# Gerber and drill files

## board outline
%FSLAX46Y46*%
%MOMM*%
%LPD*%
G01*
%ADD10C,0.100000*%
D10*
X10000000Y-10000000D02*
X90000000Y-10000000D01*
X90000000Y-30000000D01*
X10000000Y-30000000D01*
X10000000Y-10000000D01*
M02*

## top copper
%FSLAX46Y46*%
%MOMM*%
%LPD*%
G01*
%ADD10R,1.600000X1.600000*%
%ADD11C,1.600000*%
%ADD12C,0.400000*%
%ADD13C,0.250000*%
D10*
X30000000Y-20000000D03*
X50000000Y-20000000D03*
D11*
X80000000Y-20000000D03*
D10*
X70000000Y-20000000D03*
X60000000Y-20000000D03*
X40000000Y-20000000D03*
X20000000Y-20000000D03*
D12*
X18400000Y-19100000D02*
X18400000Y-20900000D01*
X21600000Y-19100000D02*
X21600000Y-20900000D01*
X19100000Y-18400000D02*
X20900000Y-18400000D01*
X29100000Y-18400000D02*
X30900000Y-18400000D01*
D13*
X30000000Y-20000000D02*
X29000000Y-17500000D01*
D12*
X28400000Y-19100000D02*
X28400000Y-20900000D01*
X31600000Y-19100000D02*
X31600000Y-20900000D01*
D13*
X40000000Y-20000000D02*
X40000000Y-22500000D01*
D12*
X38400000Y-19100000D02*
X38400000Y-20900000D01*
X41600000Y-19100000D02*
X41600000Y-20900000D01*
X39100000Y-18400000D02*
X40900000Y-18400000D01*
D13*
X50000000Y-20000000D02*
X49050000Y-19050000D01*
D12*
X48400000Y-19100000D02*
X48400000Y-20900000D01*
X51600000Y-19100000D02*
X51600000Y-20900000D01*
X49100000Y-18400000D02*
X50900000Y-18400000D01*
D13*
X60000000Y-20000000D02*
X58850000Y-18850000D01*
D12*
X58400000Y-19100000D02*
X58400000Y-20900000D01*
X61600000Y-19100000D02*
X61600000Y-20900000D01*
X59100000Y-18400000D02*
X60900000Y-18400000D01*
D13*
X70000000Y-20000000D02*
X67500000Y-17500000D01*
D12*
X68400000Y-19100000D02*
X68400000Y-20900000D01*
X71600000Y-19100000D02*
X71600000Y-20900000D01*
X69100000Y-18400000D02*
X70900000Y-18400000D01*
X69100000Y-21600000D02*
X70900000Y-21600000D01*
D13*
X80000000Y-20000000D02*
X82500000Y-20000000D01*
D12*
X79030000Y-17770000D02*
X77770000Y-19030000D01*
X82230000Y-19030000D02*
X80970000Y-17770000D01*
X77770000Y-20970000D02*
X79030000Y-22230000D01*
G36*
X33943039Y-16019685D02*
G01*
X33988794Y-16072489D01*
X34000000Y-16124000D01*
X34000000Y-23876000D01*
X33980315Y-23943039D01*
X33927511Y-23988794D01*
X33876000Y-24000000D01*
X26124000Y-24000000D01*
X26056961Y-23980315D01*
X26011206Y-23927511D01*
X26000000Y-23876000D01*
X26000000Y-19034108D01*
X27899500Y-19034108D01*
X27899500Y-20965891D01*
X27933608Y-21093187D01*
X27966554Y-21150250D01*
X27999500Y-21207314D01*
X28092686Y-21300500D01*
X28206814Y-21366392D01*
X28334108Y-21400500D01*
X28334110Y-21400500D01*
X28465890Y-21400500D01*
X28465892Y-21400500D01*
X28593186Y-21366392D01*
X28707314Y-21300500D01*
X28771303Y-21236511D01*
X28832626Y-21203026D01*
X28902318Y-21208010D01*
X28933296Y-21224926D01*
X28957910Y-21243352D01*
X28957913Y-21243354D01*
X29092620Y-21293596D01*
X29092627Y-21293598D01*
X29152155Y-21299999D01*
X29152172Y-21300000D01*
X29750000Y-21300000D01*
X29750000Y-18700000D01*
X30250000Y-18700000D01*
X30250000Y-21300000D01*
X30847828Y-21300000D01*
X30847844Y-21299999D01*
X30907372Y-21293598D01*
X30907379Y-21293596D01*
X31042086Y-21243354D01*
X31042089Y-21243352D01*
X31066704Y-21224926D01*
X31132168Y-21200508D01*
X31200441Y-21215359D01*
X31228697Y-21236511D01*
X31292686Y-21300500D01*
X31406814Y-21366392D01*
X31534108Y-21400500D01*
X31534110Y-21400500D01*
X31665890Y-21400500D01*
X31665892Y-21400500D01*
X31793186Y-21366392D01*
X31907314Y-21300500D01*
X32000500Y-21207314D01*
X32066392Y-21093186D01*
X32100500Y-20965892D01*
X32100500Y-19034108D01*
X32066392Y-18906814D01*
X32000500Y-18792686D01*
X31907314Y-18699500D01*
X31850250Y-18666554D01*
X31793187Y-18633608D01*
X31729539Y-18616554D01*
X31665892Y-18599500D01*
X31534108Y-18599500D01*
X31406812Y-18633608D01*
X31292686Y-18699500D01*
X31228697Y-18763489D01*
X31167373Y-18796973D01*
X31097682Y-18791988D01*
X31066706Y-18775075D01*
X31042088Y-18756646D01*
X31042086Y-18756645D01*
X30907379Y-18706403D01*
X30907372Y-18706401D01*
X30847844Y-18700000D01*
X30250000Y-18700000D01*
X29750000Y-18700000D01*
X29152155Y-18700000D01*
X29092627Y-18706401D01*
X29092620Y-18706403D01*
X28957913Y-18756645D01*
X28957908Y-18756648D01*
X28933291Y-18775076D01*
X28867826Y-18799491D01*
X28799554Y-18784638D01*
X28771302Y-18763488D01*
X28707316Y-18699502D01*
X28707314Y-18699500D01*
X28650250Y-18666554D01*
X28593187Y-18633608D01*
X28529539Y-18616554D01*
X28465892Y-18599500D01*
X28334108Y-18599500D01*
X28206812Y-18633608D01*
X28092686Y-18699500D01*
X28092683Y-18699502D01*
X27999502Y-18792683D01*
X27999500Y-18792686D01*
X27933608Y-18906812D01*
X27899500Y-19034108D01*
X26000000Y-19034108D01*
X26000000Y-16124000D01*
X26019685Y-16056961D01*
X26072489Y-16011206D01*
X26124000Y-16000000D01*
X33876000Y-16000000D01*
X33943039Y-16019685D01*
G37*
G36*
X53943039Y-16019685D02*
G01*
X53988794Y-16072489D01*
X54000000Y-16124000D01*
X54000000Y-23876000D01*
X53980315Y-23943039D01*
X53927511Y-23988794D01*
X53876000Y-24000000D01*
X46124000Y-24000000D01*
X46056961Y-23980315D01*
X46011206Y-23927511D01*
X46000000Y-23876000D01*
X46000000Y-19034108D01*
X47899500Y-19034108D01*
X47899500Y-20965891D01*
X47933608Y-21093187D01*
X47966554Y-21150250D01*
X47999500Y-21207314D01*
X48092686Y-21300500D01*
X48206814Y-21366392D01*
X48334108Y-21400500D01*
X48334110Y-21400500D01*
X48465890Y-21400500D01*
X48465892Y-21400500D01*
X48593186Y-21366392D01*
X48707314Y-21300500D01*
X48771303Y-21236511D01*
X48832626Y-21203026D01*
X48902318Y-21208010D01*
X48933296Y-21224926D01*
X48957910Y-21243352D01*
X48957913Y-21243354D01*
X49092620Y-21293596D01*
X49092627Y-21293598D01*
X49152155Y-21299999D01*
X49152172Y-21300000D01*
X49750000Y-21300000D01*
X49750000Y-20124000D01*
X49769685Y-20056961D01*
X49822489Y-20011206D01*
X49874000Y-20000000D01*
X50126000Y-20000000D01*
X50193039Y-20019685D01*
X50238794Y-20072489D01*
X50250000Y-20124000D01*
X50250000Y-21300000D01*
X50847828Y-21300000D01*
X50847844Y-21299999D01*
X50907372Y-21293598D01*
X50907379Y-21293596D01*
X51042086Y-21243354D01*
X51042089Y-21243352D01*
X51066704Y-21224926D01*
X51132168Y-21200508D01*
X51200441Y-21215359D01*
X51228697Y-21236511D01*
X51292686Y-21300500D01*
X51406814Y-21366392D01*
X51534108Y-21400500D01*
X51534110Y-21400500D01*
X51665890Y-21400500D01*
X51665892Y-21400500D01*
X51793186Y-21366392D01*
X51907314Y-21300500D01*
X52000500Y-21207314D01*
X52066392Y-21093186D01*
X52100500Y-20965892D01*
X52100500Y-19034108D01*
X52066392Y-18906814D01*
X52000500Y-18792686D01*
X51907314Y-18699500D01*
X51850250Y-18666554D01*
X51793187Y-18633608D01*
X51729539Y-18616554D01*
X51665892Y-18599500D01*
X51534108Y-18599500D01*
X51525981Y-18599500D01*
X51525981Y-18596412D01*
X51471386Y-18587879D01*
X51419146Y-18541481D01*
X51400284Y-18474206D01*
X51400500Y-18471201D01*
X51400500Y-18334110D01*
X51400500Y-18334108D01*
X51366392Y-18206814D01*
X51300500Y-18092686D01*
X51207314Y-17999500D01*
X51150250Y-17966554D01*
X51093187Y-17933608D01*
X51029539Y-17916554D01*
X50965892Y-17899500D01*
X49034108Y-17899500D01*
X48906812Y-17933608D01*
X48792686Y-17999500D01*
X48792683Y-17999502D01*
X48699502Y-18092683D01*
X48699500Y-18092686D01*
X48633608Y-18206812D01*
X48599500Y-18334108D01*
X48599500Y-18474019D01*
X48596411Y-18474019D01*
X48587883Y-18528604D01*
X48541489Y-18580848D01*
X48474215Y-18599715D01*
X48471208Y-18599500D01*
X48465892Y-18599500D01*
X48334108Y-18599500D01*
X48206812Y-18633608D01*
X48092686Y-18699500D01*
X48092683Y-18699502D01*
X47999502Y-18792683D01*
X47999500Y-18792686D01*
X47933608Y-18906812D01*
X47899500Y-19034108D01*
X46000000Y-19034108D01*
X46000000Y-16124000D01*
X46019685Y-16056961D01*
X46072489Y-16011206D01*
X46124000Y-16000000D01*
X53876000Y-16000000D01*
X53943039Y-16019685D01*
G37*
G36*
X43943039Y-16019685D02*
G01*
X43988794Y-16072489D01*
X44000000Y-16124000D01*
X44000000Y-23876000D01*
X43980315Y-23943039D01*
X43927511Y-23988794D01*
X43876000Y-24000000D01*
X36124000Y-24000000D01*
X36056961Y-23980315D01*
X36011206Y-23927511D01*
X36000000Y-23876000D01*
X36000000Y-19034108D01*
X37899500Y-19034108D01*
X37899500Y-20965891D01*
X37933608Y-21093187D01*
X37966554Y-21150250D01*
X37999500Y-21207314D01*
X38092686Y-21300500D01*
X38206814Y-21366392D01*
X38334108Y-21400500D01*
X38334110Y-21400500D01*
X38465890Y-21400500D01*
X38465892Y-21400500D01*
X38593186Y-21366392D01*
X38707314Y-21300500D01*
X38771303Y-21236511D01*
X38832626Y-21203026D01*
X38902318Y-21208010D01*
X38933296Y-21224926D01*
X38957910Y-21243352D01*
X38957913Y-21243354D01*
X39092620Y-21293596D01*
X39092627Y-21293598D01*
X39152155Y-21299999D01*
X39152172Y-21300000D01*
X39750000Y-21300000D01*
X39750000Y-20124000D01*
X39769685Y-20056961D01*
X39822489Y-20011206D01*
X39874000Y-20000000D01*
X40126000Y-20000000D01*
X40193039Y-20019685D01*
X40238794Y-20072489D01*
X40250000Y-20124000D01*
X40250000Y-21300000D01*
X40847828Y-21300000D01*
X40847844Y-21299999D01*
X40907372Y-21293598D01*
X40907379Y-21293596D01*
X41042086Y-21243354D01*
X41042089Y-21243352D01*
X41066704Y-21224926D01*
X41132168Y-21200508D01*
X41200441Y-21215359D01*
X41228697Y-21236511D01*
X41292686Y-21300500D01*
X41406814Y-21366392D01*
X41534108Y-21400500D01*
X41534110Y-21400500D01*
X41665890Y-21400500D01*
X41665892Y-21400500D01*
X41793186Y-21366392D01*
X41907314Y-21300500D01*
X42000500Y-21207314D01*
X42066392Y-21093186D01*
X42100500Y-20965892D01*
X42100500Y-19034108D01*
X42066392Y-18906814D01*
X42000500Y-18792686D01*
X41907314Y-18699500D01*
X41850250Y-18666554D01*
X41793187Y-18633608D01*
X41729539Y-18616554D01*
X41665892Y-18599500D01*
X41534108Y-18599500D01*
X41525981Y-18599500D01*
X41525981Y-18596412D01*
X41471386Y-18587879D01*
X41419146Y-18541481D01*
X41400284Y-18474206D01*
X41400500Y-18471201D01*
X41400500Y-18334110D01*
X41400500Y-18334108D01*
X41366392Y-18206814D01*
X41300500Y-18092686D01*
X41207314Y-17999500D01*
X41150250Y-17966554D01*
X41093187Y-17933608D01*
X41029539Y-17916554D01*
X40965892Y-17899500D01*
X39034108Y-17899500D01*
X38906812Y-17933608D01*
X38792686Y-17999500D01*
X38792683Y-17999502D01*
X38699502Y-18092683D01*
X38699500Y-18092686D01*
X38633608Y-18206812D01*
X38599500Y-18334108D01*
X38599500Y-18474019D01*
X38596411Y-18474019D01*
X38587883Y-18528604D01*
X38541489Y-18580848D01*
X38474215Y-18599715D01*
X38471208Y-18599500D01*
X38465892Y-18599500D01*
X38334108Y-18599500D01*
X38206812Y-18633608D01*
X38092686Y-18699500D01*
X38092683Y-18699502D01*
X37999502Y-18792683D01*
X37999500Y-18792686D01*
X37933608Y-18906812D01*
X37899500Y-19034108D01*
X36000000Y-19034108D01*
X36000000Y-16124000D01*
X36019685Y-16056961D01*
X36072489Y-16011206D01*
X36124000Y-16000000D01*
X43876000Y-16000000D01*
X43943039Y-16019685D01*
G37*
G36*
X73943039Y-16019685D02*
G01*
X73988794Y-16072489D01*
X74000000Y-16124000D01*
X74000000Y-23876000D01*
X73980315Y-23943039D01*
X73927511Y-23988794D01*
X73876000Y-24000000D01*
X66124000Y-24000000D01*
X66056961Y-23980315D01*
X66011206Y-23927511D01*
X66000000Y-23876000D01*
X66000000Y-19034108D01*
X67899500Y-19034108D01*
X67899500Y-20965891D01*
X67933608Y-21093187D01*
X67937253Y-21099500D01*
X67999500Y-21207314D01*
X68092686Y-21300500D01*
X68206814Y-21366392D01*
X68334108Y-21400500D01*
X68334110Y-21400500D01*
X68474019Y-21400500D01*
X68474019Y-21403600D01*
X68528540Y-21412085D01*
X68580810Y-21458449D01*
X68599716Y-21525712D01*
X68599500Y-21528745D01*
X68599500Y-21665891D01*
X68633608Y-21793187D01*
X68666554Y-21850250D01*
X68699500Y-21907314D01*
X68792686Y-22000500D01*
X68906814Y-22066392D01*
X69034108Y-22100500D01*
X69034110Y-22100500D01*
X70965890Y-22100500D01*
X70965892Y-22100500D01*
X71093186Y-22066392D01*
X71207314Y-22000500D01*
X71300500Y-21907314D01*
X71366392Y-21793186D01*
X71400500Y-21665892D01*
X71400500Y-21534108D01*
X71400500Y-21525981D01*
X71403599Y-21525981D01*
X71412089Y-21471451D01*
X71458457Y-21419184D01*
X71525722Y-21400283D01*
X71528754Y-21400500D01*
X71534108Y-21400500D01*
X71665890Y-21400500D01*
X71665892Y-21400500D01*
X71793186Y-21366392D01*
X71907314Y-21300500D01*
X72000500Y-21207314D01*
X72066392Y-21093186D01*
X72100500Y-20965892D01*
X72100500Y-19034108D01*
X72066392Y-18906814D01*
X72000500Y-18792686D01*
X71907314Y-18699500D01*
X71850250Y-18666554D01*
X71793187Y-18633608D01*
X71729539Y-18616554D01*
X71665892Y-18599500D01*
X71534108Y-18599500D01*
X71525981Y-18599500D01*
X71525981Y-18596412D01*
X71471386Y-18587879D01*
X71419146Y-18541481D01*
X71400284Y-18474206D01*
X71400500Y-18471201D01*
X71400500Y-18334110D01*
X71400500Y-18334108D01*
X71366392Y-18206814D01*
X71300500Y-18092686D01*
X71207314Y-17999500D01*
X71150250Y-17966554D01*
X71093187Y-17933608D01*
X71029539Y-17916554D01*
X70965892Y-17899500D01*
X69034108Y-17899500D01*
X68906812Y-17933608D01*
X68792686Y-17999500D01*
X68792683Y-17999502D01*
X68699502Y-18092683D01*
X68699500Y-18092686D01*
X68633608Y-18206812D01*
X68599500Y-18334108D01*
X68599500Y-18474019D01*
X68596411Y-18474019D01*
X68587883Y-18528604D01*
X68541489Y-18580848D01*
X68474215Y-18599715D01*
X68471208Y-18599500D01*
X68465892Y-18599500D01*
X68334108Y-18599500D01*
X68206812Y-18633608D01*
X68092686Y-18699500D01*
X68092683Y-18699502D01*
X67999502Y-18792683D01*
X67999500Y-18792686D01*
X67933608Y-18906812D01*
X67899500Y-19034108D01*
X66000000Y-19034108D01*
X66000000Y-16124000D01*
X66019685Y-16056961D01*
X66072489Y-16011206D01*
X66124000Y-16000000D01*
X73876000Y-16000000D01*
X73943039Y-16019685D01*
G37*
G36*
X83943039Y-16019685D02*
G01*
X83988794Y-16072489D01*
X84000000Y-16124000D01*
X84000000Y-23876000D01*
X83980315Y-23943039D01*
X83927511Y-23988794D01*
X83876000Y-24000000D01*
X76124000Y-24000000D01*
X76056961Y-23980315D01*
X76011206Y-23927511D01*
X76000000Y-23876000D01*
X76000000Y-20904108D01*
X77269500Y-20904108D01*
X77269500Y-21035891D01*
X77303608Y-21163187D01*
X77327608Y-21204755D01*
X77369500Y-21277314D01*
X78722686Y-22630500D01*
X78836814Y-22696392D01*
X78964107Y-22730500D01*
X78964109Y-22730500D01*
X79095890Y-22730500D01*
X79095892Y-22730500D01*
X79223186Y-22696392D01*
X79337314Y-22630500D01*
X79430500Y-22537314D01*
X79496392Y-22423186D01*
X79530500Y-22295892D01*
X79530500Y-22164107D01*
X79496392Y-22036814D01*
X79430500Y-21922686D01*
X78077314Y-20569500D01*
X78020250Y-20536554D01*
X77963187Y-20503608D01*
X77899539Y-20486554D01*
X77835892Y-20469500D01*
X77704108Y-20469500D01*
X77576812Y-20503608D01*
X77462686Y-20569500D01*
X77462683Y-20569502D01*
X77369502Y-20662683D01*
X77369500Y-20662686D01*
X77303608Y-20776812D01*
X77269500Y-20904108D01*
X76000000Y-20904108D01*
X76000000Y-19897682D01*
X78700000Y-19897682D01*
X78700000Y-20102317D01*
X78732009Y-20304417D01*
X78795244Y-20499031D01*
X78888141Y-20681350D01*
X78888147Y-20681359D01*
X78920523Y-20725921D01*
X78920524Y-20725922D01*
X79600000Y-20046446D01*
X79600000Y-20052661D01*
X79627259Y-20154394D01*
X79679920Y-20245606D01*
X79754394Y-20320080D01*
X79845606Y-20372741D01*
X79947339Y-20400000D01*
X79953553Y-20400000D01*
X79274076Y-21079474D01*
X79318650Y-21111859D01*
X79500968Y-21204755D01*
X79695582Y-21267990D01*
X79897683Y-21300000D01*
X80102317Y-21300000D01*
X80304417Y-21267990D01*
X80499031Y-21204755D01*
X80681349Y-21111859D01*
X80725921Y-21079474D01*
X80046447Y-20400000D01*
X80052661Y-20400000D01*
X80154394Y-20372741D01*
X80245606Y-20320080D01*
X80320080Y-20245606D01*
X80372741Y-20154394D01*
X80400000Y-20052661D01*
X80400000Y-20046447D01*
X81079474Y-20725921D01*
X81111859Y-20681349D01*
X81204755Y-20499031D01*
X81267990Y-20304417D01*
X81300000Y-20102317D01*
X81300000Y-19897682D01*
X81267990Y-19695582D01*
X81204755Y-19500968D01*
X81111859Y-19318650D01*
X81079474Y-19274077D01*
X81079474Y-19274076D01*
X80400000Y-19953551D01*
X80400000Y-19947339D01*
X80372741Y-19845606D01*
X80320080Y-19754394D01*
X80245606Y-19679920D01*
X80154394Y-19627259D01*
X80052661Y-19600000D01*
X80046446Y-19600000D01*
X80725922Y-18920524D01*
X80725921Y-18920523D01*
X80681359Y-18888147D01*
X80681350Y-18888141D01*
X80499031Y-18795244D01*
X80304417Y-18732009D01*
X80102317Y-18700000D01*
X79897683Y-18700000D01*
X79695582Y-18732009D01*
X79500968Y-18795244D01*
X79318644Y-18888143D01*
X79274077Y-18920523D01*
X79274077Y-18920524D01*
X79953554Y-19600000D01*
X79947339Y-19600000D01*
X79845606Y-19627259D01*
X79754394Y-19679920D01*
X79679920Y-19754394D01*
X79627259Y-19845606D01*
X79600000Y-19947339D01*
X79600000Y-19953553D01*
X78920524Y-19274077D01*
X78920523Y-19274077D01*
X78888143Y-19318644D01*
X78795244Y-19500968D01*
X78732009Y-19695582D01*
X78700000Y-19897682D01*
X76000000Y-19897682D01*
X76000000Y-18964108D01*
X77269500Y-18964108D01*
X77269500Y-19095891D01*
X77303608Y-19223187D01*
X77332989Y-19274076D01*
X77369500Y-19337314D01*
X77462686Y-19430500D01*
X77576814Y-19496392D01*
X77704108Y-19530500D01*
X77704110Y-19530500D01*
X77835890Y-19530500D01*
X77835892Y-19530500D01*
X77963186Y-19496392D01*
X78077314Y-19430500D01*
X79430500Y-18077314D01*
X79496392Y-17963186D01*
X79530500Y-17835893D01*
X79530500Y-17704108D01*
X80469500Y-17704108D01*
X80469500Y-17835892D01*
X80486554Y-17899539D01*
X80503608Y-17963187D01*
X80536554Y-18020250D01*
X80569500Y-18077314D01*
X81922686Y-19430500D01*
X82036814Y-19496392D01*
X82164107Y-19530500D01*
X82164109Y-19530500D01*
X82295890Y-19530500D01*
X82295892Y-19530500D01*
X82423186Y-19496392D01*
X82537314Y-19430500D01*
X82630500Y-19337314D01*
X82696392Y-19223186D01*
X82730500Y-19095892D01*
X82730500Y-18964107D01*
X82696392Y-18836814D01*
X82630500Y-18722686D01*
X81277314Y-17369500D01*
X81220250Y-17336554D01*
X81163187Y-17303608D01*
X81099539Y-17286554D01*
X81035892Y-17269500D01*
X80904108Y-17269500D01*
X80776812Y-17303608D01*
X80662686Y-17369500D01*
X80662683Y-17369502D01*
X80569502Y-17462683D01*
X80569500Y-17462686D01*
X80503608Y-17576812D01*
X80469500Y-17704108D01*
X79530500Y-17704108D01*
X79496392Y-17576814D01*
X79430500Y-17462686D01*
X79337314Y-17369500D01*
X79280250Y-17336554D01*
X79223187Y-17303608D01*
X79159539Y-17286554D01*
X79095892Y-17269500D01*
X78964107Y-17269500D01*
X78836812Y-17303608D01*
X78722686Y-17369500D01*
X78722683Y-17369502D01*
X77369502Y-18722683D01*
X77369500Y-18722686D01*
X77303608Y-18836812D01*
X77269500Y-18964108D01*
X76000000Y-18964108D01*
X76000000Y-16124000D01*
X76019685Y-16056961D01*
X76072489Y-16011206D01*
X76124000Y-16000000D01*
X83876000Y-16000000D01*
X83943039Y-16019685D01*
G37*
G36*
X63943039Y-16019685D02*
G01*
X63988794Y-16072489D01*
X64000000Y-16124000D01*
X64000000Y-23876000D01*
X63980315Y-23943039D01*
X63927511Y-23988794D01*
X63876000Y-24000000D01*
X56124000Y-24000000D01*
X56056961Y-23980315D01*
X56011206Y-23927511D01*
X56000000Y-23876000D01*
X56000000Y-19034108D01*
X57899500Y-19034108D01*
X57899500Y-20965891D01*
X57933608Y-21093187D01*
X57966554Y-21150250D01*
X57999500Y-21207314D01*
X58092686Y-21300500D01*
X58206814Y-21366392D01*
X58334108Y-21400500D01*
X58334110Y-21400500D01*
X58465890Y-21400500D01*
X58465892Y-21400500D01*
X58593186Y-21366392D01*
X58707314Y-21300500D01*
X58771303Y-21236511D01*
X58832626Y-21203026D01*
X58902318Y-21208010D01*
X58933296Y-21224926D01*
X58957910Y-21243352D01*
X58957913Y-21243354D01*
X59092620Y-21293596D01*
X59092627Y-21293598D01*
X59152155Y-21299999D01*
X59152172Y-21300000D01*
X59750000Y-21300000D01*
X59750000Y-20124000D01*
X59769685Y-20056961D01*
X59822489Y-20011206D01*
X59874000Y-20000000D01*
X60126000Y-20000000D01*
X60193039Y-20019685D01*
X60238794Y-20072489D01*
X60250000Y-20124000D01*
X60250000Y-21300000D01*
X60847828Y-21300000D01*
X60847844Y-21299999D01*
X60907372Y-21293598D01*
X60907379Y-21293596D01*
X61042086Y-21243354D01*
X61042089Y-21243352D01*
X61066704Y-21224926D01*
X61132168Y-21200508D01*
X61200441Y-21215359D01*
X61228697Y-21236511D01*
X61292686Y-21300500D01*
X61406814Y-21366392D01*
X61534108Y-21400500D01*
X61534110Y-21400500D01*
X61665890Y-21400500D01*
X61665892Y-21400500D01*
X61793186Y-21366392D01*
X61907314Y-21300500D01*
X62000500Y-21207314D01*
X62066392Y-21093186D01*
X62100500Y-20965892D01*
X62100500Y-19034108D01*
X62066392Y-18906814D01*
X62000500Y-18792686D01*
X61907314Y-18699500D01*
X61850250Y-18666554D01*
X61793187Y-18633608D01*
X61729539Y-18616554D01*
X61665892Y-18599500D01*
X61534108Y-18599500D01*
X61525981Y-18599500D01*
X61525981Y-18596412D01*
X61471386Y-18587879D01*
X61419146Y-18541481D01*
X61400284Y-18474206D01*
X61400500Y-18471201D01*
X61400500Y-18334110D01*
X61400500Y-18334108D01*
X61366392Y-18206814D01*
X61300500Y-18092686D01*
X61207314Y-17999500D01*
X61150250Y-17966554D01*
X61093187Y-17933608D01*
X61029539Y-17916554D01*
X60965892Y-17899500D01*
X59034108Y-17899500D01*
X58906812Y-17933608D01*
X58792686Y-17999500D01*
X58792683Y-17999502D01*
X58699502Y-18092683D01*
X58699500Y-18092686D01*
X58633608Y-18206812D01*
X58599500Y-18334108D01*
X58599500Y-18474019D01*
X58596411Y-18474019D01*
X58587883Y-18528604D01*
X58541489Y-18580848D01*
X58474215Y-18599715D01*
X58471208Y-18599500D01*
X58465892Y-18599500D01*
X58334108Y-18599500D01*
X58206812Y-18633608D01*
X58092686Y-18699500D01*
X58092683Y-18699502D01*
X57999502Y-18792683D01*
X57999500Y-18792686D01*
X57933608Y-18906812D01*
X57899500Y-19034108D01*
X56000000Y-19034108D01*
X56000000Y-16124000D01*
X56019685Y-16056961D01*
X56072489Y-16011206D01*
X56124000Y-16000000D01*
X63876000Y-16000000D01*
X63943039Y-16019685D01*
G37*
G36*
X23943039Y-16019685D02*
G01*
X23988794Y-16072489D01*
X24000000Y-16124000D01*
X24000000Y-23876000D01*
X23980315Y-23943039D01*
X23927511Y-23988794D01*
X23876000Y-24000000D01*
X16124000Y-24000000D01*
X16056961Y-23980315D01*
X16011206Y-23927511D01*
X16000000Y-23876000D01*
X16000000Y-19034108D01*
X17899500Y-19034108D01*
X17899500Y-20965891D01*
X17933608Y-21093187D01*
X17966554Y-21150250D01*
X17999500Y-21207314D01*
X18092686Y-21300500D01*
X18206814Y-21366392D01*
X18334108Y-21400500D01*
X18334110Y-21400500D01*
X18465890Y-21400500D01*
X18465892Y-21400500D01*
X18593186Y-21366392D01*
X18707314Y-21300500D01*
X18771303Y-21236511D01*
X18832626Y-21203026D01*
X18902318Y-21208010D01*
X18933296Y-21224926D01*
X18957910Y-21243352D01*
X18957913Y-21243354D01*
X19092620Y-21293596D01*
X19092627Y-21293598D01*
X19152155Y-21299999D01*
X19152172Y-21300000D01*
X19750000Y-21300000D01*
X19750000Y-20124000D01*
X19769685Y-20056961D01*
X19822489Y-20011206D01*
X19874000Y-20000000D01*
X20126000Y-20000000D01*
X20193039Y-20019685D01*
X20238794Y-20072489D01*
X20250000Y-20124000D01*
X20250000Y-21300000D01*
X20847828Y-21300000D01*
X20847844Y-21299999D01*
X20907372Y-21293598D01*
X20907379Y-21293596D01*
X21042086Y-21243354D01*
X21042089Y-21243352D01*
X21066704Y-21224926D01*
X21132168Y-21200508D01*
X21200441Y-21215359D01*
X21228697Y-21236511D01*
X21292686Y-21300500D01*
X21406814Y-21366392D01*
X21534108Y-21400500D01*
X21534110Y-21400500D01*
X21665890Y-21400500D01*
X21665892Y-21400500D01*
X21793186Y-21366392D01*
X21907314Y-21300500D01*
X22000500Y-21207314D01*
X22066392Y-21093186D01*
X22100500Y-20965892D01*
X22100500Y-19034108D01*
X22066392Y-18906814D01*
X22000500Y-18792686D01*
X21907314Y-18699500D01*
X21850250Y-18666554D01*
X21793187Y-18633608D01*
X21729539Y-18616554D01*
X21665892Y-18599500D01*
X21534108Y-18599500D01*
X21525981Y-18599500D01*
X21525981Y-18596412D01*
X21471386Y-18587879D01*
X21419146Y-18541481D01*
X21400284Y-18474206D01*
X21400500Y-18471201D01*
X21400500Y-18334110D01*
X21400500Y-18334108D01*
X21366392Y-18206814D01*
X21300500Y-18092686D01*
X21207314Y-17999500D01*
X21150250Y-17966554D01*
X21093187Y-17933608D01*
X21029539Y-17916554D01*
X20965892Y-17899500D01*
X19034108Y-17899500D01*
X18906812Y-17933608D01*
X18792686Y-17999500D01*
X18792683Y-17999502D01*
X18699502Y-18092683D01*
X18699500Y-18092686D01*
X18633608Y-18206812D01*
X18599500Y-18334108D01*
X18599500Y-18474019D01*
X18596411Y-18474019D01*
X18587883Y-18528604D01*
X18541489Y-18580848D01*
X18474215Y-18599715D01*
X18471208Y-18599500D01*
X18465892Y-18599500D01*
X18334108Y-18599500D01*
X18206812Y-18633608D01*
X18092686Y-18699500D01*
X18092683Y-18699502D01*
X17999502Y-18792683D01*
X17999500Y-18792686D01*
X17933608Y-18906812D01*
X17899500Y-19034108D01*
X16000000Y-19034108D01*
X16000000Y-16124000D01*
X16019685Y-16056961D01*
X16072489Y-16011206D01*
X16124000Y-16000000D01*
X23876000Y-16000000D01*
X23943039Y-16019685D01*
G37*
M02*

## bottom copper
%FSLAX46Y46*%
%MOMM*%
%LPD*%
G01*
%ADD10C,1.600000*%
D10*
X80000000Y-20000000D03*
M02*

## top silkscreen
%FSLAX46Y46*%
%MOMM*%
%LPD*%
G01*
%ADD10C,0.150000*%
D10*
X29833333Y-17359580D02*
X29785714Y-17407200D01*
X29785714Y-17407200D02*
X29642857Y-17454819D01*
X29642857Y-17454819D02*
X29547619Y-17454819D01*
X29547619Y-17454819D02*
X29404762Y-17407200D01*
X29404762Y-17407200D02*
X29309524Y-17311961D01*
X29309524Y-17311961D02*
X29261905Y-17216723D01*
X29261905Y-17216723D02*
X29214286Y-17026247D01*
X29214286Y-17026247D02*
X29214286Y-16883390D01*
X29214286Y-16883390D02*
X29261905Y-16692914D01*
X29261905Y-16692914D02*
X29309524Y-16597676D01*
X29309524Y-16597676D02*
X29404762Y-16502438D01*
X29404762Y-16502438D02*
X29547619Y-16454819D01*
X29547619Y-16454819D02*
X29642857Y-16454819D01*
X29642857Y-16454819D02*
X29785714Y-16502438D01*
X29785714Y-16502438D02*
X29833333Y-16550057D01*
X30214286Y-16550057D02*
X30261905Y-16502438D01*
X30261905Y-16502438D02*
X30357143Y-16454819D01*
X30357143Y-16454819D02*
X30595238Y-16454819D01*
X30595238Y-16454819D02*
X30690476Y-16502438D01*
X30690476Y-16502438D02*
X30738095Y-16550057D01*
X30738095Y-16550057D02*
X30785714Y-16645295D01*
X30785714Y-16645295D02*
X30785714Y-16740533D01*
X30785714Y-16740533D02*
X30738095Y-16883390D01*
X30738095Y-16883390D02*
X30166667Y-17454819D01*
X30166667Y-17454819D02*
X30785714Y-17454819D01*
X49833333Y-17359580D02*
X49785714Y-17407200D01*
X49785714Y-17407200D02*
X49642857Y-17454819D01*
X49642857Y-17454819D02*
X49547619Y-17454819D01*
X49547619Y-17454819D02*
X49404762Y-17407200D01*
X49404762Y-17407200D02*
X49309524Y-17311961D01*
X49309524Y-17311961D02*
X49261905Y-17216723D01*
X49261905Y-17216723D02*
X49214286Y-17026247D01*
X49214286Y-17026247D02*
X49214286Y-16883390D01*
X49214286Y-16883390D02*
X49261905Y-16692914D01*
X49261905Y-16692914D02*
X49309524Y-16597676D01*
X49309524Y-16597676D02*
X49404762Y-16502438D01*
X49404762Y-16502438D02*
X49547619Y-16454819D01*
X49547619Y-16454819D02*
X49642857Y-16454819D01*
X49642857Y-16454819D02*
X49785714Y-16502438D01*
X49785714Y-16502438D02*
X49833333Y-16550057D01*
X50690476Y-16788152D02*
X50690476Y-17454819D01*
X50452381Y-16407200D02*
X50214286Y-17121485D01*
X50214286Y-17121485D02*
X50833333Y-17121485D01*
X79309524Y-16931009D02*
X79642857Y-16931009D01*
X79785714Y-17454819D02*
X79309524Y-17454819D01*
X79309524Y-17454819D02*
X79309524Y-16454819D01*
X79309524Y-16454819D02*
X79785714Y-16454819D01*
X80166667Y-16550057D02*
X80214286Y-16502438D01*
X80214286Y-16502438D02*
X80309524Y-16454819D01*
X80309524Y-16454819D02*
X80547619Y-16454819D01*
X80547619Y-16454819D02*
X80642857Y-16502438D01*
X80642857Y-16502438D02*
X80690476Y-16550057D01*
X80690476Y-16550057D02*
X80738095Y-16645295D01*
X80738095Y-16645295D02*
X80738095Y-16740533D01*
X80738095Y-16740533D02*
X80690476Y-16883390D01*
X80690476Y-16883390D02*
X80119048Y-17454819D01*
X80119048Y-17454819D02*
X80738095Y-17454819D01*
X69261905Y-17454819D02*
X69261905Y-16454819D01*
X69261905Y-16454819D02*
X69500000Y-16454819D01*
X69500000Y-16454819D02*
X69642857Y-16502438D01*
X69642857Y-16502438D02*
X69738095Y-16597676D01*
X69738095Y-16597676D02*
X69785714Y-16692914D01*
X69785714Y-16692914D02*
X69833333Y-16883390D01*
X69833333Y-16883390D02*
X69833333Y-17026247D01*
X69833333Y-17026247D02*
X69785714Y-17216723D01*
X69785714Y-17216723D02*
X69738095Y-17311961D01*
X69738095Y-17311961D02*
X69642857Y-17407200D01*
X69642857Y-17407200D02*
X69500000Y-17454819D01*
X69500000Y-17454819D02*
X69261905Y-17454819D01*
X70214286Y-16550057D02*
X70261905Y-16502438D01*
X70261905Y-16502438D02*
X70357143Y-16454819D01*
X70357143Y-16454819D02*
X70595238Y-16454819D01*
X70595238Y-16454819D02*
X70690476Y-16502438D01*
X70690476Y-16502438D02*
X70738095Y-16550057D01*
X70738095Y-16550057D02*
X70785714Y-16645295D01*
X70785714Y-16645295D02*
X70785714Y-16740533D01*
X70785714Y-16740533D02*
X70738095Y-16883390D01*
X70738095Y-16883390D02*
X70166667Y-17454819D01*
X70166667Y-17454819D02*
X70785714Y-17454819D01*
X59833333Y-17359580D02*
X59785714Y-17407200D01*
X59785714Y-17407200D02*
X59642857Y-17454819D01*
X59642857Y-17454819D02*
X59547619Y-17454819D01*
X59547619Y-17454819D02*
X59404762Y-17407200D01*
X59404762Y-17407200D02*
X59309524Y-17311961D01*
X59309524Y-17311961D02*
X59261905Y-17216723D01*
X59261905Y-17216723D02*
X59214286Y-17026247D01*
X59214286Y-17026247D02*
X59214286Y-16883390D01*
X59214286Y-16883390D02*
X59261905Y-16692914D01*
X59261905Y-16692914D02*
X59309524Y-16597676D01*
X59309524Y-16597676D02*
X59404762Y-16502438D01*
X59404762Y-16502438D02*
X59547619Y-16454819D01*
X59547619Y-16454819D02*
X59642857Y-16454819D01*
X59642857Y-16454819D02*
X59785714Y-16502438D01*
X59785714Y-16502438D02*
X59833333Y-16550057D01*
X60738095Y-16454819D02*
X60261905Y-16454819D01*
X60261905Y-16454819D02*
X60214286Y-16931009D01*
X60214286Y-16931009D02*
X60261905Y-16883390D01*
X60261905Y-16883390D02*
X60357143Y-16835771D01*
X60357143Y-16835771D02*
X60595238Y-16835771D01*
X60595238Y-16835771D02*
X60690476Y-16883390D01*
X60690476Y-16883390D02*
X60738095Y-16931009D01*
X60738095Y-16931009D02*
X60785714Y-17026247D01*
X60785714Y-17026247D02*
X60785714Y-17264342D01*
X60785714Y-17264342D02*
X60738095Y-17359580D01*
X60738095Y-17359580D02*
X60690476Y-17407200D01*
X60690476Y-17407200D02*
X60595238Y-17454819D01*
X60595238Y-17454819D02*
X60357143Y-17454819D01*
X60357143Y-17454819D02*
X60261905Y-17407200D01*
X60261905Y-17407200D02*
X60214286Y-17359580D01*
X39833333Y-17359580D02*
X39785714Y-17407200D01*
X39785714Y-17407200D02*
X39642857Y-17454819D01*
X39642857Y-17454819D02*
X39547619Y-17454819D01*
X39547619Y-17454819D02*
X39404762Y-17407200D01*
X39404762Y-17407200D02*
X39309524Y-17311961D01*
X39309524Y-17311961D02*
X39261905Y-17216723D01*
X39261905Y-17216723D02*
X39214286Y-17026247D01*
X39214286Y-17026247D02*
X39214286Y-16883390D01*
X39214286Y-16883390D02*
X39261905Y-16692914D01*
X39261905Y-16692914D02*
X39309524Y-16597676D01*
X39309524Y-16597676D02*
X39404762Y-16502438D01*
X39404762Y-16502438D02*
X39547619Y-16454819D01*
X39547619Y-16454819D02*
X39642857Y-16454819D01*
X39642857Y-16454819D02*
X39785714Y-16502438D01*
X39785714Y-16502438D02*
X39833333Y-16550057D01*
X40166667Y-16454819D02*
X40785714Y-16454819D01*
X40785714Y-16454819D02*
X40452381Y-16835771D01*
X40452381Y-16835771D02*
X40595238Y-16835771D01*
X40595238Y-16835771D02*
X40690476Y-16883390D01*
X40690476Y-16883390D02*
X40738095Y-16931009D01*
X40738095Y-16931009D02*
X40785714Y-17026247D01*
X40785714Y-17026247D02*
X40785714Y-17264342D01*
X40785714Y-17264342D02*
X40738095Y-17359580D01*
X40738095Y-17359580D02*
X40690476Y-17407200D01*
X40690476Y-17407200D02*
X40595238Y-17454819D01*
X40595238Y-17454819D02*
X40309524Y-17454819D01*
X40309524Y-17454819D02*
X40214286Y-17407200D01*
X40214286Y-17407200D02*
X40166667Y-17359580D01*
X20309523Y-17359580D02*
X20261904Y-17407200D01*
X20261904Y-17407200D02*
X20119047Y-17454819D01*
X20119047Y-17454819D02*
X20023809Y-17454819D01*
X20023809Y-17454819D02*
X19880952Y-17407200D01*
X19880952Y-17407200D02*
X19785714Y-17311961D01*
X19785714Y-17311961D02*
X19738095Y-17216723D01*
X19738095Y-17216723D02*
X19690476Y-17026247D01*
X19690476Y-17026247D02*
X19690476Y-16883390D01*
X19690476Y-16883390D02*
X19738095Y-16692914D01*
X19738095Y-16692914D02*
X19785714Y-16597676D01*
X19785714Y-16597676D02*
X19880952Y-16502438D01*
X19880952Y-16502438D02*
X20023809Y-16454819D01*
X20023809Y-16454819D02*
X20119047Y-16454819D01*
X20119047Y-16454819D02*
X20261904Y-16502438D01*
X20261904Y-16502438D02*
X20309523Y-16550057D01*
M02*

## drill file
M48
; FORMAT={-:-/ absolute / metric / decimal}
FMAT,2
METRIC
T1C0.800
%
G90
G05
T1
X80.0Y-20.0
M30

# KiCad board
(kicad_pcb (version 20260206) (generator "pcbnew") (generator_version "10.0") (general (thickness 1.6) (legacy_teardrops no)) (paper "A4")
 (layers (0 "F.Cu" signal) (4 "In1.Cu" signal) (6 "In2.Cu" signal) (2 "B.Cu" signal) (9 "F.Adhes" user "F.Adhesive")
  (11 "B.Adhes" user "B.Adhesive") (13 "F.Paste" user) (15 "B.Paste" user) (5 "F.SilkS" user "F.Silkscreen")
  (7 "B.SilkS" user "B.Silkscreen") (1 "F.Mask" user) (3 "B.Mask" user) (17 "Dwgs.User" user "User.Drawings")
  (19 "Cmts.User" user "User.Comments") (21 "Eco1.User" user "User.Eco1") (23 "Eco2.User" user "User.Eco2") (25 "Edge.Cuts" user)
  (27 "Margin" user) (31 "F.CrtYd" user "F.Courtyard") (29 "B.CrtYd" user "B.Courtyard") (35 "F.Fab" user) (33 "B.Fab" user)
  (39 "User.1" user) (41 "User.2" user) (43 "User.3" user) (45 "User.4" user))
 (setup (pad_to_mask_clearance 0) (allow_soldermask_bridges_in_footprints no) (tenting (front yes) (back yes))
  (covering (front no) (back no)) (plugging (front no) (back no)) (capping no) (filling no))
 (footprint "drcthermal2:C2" (layer "F.Cu") (at 30 20)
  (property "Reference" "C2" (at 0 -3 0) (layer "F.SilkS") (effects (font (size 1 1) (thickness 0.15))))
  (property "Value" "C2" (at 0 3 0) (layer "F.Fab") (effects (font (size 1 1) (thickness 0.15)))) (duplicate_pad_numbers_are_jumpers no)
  (pad "1" smd rect (at 0 0) (size 1.6 1.6) (layers "F.Cu" "F.Mask" "F.Paste") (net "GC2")))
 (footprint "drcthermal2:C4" (layer "F.Cu") (at 50 20)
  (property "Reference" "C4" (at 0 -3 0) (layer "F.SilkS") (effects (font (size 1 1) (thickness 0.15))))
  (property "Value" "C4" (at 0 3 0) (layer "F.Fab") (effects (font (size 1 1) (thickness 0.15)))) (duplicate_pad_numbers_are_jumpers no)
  (pad "1" smd rect (at 0 0) (size 1.6 1.6) (layers "F.Cu" "F.Mask" "F.Paste") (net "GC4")))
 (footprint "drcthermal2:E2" (layer "F.Cu") (at 80 20)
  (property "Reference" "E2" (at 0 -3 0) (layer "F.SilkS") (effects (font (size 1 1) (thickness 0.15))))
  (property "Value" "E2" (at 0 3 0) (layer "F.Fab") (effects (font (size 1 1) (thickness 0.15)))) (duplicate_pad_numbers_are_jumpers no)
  (pad "1" thru_hole circle (at 0 0) (size 1.6 1.6) (drill 0.8) (layers "*.Cu" "*.Mask") (remove_unused_layers no) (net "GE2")))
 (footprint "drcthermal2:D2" (layer "F.Cu") (at 70 20)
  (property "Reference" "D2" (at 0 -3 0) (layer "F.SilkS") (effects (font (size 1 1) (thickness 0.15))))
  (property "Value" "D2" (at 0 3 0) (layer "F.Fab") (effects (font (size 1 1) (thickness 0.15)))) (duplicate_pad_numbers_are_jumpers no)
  (pad "1" smd rect (at 0 0) (size 1.6 1.6) (layers "F.Cu" "F.Mask" "F.Paste") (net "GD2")))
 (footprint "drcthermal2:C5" (layer "F.Cu") (at 60 20)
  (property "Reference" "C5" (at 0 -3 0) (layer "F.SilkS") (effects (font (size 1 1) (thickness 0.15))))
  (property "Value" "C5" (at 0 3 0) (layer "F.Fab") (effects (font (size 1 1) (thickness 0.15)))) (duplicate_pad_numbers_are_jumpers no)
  (pad "1" smd rect (at 0 0) (size 1.6 1.6) (layers "F.Cu" "F.Mask" "F.Paste") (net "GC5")))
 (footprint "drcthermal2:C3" (layer "F.Cu") (at 40 20)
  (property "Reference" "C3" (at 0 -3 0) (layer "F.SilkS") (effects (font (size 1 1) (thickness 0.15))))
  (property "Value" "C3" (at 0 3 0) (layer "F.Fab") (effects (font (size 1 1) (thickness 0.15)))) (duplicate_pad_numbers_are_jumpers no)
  (pad "1" smd rect (at 0 0) (size 1.6 1.6) (layers "F.Cu" "F.Mask" "F.Paste") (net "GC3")))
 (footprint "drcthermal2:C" (layer "F.Cu") (at 20 20)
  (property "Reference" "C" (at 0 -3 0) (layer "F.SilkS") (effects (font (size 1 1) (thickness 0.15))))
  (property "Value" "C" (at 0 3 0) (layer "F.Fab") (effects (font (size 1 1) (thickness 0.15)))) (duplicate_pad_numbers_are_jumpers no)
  (pad "1" smd rect (at 0 0) (size 1.6 1.6) (layers "F.Cu" "F.Mask" "F.Paste") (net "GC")))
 (gr_rect (start 10 10) (end 90 30) (stroke (width 0.1) (type solid)) (fill no) (layer "Edge.Cuts"))
 (segment (start 18.4 19.1) (end 18.4 20.9) (width 0.4) (layer "F.Cu") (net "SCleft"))
 (segment (start 21.6 19.1) (end 21.6 20.9) (width 0.4) (layer "F.Cu") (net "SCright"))
 (segment (start 19.1 18.4) (end 20.9 18.4) (width 0.4) (layer "F.Cu") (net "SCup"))
 (segment (start 29.1 18.4) (end 30.9 18.4) (width 0.4) (layer "F.Cu") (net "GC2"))
 (segment (start 30 20) (end 29 17.5) (width 0.25) (layer "F.Cu") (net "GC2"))
 (segment (start 28.4 19.1) (end 28.4 20.9) (width 0.4) (layer "F.Cu") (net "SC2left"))
 (segment (start 31.6 19.1) (end 31.6 20.9) (width 0.4) (layer "F.Cu") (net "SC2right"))
 (segment (start 40 20) (end 40 22.5) (width 0.25) (layer "F.Cu") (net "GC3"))
 (segment (start 38.4 19.1) (end 38.4 20.9) (width 0.4) (layer "F.Cu") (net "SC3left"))
 (segment (start 41.6 19.1) (end 41.6 20.9) (width 0.4) (layer "F.Cu") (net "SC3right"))
 (segment (start 39.1 18.4) (end 40.9 18.4) (width 0.4) (layer "F.Cu") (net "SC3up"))
 (segment (start 50 20) (end 49.05 19.05) (width 0.25) (layer "F.Cu") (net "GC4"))
 (segment (start 48.4 19.1) (end 48.4 20.9) (width 0.4) (layer "F.Cu") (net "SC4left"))
 (segment (start 51.6 19.1) (end 51.6 20.9) (width 0.4) (layer "F.Cu") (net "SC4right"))
 (segment (start 49.1 18.4) (end 50.9 18.4) (width 0.4) (layer "F.Cu") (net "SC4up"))
 (segment (start 60 20) (end 58.85 18.85) (width 0.25) (layer "F.Cu") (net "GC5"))
 (segment (start 58.4 19.1) (end 58.4 20.9) (width 0.4) (layer "F.Cu") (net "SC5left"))
 (segment (start 61.6 19.1) (end 61.6 20.9) (width 0.4) (layer "F.Cu") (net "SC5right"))
 (segment (start 59.1 18.4) (end 60.9 18.4) (width 0.4) (layer "F.Cu") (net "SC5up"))
 (segment (start 70 20) (end 67.5 17.5) (width 0.25) (layer "F.Cu") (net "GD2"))
 (segment (start 68.4 19.1) (end 68.4 20.9) (width 0.4) (layer "F.Cu") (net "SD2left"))
 (segment (start 71.6 19.1) (end 71.6 20.9) (width 0.4) (layer "F.Cu") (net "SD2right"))
 (segment (start 69.1 18.4) (end 70.9 18.4) (width 0.4) (layer "F.Cu") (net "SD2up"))
 (segment (start 69.1 21.6) (end 70.9 21.6) (width 0.4) (layer "F.Cu") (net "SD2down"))
 (segment (start 80 20) (end 82.5 20) (width 0.25) (layer "F.Cu") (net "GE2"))
 (segment (start 79.03 17.77) (end 77.77 19.03) (width 0.4) (layer "F.Cu") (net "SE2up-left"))
 (segment (start 82.23 19.03) (end 80.97 17.77) (width 0.4) (layer "F.Cu") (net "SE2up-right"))
 (segment (start 77.77 20.97) (end 79.03 22.23) (width 0.4) (layer "F.Cu") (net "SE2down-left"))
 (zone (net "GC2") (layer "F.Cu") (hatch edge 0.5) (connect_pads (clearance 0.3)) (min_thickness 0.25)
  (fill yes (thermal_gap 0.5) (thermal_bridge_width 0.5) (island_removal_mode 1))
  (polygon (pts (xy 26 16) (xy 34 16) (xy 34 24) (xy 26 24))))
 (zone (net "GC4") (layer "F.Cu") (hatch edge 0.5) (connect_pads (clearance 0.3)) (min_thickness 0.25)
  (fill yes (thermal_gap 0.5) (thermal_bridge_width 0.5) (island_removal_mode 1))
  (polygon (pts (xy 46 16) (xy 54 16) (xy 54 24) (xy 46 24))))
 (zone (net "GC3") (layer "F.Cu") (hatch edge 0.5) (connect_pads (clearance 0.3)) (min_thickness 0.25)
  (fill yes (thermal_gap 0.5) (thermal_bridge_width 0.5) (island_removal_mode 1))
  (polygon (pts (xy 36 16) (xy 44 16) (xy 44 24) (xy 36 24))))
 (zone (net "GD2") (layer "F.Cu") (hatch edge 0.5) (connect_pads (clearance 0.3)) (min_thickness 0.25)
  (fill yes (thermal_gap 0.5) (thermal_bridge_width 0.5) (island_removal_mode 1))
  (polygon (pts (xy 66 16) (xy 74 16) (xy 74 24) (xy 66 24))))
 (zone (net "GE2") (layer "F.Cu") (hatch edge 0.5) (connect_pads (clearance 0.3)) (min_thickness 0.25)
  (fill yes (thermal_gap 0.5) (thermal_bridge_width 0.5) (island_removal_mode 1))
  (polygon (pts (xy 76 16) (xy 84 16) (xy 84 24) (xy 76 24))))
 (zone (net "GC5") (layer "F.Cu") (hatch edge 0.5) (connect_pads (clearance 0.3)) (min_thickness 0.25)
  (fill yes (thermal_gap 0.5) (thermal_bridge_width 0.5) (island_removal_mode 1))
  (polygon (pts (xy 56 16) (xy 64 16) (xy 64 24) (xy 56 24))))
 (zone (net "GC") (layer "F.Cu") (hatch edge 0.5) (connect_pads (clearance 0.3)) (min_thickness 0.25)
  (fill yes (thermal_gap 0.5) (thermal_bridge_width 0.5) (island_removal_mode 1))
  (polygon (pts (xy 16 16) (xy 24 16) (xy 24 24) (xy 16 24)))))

